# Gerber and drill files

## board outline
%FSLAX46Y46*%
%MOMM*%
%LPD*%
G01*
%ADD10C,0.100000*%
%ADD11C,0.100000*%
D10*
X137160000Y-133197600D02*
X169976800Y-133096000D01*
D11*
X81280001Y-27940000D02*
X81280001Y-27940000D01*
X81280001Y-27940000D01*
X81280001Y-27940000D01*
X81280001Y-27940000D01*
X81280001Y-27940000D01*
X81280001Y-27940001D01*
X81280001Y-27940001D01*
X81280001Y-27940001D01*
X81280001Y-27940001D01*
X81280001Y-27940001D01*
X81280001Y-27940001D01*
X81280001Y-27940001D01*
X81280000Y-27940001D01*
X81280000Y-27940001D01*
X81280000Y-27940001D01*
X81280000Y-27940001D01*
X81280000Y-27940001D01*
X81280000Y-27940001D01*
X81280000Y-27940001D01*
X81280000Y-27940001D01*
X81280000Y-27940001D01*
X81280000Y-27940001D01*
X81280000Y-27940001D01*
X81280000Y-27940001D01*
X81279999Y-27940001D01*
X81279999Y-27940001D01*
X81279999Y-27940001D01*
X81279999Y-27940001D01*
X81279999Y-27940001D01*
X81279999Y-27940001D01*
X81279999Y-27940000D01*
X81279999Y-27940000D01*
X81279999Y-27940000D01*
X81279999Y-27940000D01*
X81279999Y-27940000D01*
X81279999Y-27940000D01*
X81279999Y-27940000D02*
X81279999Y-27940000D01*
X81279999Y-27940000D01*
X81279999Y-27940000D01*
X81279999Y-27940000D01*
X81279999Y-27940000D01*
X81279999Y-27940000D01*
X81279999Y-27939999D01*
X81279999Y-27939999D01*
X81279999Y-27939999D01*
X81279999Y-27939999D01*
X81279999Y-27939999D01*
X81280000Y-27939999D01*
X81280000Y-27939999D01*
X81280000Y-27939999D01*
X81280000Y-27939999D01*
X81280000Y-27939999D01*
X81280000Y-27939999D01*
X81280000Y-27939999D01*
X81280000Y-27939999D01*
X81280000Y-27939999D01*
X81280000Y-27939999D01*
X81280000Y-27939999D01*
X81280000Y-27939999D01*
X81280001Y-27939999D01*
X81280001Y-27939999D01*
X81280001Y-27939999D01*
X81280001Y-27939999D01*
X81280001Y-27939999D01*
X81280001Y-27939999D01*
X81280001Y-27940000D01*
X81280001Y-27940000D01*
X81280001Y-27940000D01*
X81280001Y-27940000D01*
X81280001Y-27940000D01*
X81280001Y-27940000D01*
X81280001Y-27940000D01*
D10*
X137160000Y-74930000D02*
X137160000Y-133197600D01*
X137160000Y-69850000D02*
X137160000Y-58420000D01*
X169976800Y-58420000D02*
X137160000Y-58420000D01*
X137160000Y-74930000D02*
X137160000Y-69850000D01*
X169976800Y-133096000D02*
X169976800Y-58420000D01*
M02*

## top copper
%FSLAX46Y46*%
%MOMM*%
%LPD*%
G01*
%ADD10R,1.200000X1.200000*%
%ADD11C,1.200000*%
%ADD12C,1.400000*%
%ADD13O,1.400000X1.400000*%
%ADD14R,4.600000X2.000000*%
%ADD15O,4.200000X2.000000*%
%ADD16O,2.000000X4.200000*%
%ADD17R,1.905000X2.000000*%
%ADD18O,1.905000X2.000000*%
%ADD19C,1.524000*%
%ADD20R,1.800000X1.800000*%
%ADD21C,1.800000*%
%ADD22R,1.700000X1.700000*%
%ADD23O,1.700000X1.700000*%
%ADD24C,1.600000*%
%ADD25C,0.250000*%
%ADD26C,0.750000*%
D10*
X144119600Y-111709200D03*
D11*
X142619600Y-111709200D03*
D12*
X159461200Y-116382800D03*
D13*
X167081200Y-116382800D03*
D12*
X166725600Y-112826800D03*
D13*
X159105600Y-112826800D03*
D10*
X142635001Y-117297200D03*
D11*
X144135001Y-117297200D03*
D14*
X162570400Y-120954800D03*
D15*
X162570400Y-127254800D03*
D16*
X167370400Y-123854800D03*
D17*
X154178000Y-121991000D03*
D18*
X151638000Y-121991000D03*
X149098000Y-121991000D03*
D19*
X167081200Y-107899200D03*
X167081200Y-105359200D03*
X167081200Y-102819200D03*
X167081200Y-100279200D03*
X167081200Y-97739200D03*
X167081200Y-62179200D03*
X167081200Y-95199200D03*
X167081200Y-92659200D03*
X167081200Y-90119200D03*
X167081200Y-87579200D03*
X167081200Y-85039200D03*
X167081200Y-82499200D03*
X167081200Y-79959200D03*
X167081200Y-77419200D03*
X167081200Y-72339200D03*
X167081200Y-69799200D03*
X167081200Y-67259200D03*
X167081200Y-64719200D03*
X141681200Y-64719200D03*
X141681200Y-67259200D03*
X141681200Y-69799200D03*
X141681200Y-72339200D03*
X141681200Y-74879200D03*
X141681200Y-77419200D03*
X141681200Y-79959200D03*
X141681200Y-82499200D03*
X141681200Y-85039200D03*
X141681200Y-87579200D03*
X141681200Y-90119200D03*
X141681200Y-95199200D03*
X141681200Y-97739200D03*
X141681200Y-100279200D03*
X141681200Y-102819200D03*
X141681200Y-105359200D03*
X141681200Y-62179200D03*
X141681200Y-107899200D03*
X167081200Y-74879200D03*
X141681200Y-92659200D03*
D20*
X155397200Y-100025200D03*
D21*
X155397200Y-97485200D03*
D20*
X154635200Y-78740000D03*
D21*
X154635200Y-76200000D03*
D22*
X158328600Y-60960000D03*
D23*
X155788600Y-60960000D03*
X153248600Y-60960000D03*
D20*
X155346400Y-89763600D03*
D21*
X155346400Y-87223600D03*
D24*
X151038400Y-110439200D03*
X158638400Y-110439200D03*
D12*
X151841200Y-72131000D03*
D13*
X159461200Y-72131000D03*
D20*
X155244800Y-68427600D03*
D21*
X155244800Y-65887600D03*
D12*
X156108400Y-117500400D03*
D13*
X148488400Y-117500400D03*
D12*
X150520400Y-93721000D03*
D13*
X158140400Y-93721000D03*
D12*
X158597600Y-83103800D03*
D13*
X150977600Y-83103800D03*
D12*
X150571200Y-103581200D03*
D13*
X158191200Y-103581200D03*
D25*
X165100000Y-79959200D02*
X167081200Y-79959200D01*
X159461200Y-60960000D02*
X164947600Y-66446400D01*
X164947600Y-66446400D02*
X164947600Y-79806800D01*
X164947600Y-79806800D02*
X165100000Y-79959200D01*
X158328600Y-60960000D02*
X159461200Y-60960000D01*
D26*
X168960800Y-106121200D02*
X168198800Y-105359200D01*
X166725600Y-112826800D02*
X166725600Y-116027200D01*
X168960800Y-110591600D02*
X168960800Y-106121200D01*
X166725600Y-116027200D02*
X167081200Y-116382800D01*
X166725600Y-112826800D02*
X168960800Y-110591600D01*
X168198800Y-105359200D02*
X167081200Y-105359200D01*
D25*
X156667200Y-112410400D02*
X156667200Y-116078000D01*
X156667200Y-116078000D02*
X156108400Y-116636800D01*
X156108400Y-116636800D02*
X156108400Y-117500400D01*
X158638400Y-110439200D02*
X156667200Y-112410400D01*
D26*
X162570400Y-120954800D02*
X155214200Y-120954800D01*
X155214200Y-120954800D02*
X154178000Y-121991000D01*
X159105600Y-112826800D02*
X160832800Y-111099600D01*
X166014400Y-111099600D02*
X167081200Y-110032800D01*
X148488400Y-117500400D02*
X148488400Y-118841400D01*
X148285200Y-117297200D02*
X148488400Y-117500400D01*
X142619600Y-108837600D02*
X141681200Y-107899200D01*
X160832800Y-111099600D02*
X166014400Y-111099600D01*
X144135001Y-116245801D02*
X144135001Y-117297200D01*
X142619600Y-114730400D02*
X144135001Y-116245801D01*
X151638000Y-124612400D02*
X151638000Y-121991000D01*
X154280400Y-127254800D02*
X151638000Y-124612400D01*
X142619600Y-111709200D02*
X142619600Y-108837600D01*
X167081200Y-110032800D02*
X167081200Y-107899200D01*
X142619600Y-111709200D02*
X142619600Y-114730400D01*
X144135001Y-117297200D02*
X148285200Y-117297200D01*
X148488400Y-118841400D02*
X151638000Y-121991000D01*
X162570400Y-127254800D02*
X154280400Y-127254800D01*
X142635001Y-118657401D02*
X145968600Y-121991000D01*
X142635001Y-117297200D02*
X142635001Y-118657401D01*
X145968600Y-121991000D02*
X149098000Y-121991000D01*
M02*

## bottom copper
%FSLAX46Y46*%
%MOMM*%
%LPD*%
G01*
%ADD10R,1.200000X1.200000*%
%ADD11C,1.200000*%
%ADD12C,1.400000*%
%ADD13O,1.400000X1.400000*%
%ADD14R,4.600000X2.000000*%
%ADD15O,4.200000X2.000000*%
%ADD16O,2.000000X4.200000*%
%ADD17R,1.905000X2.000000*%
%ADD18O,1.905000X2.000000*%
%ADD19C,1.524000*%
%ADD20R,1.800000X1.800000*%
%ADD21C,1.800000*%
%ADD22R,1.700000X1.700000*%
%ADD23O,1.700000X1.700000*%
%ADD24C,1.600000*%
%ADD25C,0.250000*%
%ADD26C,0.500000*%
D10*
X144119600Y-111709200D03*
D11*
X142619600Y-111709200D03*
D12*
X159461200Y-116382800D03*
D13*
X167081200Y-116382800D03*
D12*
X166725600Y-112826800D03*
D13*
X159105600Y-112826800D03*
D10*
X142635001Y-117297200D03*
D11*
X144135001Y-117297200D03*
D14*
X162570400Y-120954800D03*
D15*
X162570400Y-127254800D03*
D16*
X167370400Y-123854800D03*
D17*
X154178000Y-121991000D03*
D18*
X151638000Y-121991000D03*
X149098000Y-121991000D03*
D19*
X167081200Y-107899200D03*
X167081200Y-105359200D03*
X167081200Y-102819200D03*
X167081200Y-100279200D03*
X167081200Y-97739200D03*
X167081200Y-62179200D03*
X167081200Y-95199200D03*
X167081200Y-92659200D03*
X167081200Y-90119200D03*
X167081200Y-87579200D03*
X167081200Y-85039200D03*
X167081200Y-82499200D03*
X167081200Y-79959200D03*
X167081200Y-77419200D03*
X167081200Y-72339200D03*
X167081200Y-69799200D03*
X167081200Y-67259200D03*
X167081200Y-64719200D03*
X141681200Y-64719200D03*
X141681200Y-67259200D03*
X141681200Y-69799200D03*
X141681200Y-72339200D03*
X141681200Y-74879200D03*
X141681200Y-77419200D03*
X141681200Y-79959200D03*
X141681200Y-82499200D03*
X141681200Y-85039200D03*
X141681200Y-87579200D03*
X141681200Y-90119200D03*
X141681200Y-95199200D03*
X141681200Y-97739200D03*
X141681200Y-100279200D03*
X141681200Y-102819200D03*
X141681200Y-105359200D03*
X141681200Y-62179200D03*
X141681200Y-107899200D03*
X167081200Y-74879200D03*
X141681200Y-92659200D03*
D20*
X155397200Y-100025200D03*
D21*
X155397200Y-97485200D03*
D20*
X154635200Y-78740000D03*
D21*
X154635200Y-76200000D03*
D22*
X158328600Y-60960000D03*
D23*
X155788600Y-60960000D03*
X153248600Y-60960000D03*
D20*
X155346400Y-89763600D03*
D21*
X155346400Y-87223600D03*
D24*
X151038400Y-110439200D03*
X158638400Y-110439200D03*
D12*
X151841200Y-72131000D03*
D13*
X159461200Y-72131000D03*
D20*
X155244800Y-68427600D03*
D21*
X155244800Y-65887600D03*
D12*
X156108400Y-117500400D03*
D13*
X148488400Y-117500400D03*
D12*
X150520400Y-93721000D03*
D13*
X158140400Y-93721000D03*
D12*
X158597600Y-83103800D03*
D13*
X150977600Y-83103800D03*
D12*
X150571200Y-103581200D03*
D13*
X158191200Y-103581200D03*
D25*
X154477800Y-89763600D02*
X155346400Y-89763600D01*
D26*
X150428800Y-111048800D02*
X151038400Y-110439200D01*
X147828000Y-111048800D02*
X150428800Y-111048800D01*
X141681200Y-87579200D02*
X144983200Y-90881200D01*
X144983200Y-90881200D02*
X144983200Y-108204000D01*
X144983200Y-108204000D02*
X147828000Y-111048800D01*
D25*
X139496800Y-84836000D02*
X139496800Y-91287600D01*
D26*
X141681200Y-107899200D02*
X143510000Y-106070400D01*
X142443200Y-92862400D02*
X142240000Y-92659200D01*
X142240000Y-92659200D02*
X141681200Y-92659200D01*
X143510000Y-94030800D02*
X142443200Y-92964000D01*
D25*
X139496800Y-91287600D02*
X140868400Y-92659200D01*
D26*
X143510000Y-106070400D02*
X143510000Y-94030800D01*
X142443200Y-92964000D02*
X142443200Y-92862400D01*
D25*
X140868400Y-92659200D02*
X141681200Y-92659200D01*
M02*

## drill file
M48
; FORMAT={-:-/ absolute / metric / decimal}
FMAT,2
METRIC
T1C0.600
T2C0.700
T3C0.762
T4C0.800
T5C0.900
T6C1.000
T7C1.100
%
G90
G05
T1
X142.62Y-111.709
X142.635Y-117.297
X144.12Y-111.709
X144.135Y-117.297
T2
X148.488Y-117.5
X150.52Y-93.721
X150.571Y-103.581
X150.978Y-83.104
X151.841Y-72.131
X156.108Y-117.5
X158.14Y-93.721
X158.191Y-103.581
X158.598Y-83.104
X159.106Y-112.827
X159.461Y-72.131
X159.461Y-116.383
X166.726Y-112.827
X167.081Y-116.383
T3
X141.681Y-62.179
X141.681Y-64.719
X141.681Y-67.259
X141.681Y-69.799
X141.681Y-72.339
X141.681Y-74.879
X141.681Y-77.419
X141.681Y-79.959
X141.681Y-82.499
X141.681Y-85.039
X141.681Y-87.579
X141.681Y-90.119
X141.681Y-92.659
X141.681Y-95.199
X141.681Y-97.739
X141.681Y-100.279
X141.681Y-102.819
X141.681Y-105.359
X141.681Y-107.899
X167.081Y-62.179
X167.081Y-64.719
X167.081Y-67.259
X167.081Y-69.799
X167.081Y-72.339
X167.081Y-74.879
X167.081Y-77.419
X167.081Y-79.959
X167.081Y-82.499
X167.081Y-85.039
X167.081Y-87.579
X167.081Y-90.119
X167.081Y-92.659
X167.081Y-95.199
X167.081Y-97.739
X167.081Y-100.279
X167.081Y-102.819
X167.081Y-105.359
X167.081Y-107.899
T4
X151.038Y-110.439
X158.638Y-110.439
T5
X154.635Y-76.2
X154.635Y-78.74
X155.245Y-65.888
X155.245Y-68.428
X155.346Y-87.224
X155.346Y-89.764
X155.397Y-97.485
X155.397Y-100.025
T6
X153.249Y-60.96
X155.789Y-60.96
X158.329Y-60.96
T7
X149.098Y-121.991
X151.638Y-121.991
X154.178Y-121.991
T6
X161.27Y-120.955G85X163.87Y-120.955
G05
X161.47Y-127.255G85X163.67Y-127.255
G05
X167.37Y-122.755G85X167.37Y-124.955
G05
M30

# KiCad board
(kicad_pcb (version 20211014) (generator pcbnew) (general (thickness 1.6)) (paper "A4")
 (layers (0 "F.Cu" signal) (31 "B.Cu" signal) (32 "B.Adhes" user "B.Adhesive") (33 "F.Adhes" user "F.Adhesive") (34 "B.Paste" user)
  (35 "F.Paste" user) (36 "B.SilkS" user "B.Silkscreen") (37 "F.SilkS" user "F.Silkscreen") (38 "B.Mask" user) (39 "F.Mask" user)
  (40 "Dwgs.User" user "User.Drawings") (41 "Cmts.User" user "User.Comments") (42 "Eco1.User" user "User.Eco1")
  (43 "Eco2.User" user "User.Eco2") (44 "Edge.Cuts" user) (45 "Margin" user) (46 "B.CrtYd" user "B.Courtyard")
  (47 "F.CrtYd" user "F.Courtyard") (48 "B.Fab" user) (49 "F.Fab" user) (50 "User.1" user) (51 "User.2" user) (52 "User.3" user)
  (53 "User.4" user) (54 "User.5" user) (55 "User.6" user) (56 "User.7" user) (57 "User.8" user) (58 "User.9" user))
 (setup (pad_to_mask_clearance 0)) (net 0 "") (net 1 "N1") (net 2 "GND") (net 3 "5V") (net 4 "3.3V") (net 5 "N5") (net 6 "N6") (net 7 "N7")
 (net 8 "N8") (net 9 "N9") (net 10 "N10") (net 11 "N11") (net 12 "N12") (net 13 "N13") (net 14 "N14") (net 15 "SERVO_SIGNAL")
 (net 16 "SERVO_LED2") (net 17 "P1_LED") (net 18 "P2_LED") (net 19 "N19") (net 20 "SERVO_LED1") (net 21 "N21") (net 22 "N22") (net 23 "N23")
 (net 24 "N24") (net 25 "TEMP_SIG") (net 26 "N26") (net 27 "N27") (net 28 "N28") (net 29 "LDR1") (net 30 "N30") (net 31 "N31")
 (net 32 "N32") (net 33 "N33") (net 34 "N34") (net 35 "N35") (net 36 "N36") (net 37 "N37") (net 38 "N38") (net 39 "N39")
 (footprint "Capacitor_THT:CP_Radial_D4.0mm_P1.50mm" (layer "F.Cu") (at 144.1196 111.7092 180)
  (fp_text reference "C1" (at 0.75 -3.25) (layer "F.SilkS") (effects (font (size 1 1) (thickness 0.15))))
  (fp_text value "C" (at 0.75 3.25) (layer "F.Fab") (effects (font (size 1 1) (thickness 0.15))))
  (pad "1" thru_hole rect (at 0 0 180) (size 1.2 1.2) (drill 0.6) (layers *.Cu *.Mask) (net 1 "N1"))
  (pad "2" thru_hole circle (at 1.5 0 180) (size 1.2 1.2) (drill 0.6) (layers *.Cu *.Mask) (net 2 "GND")))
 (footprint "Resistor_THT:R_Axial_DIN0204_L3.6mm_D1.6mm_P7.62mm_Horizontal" (layer "F.Cu") (at 159.4612 116.3828)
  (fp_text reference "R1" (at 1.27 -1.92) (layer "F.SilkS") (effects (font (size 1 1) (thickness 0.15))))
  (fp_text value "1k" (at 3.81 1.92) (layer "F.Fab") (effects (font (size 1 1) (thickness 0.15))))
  (pad "1" thru_hole circle (at 0 0) (size 1.4 1.4) (drill 0.7) (layers *.Cu *.Mask) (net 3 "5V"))
  (pad "2" thru_hole oval (at 7.62 0) (size 1.4 1.4) (drill 0.7) (layers *.Cu *.Mask) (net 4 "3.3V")))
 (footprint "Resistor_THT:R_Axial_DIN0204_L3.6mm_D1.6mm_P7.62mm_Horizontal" (layer "F.Cu") (at 166.7256 112.8268 180)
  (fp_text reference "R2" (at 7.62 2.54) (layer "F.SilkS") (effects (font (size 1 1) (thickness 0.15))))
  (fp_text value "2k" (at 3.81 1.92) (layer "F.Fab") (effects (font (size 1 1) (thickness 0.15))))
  (pad "1" thru_hole circle (at 0 0 180) (size 1.4 1.4) (drill 0.7) (layers *.Cu *.Mask) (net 4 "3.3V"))
  (pad "2" thru_hole oval (at 7.62 0 180) (size 1.4 1.4) (drill 0.7) (layers *.Cu *.Mask) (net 2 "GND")))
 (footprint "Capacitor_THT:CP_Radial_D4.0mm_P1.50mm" (layer "F.Cu") (at 142.635001 117.2972)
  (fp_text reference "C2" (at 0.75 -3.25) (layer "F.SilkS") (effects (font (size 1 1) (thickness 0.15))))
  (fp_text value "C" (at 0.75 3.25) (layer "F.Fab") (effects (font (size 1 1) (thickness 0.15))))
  (pad "1" thru_hole rect (at 0 0) (size 1.2 1.2) (drill 0.6) (layers *.Cu *.Mask) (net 3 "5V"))
  (pad "2" thru_hole circle (at 1.5 0) (size 1.2 1.2) (drill 0.6) (layers *.Cu *.Mask) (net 2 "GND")))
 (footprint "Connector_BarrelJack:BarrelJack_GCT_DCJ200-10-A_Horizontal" (layer "F.Cu") (at 162.5704 120.9548)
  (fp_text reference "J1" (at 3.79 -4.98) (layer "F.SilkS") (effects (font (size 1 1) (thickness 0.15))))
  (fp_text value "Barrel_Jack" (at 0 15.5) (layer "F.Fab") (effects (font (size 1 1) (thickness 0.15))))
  (pad "1" thru_hole rect (at 0 0) (size 4.6 2) (drill oval 3.6 1) (layers *.Cu *.Mask) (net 1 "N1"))
  (pad "2" thru_hole oval (at 0 6.3) (size 4.2 2) (drill oval 3.2 1) (layers *.Cu *.Mask) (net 2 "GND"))
  (pad "3" thru_hole oval (at 4.8 2.9) (size 2 4.2) (drill oval 1 3.2) (layers *.Cu *.Mask)))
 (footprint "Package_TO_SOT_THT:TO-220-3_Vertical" (layer "F.Cu") (at 154.178 121.991 180)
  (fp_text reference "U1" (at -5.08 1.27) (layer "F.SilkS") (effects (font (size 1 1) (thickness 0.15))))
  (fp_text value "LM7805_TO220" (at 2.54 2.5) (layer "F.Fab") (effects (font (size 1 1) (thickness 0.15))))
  (pad "1" thru_hole rect (at 0 0 180) (size 1.905 2) (drill 1.1) (layers *.Cu *.Mask) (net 1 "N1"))
  (pad "2" thru_hole oval (at 2.54 0 180) (size 1.905 2) (drill 1.1) (layers *.Cu *.Mask) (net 2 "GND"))
  (pad "3" thru_hole oval (at 5.08 0 180) (size 1.905 2) (drill 1.1) (layers *.Cu *.Mask) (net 3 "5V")))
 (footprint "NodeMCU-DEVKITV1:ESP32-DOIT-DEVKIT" (layer "F.Cu") (at 154.3812 110.4392 180)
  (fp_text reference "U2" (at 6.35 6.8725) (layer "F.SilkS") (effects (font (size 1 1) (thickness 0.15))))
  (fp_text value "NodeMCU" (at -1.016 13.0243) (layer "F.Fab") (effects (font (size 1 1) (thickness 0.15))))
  (pad "1" thru_hole circle (at -12.7 2.54 180) (size 1.524 1.524) (drill 0.762) (layers *.Cu *.Mask) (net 2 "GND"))
  (pad "2" thru_hole circle (at -12.7 5.08 180) (size 1.524 1.524) (drill 0.762) (layers *.Cu *.Mask) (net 4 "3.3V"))
  (pad "3" thru_hole circle (at -12.7 7.62 180) (size 1.524 1.524) (drill 0.762) (layers *.Cu *.Mask) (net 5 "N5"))
  (pad "4" thru_hole circle (at -12.7 10.16 180) (size 1.524 1.524) (drill 0.762) (layers *.Cu *.Mask) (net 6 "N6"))
  (pad "5" thru_hole circle (at -12.7 12.7 180) (size 1.524 1.524) (drill 0.762) (layers *.Cu *.Mask) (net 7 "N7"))
  (pad "5V" thru_hole circle (at -12.7 48.26 180) (size 1.524 1.524) (drill 0.762) (layers *.Cu *.Mask) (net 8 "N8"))
  (pad "6" thru_hole circle (at -12.7 15.24 180) (size 1.524 1.524) (drill 0.762) (layers *.Cu *.Mask) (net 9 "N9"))
  (pad "7" thru_hole circle (at -12.7 17.78 180) (size 1.524 1.524) (drill 0.762) (layers *.Cu *.Mask) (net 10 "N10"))
  (pad "8" thru_hole circle (at -12.7 20.32 180) (size 1.524 1.524) (drill 0.762) (layers *.Cu *.Mask) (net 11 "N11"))
  (pad "9" thru_hole circle (at -12.7 22.86 180) (size 1.524 1.524) (drill 0.762) (layers *.Cu *.Mask) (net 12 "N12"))
  (pad "10" thru_hole circle (at -12.7 25.4 180) (size 1.524 1.524) (drill 0.762) (layers *.Cu *.Mask) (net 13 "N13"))
  (pad "11" thru_hole circle (at -12.7 27.94 180) (size 1.524 1.524) (drill 0.762) (layers *.Cu *.Mask) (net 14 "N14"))
  (pad "12" thru_hole circle (at -12.7 30.48 180) (size 1.524 1.524) (drill 0.762) (layers *.Cu *.Mask) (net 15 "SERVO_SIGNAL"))
  (pad "13" thru_hole circle (at -12.7 33.02 180) (size 1.524 1.524) (drill 0.762) (layers *.Cu *.Mask) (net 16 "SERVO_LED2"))
  (pad "15" thru_hole circle (at -12.7 38.1 180) (size 1.524 1.524) (drill 0.762) (layers *.Cu *.Mask))
  (pad "16" thru_hole circle (at -12.7 40.64 180) (size 1.524 1.524) (drill 0.762) (layers *.Cu *.Mask) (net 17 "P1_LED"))
  (pad "17" thru_hole circle (at -12.7 43.18 180) (size 1.524 1.524) (drill 0.762) (layers *.Cu *.Mask) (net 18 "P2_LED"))
  (pad "18" thru_hole circle (at -12.7 45.72 180) (size 1.524 1.524) (drill 0.762) (layers *.Cu *.Mask) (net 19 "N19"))
  (pad "19" thru_hole circle (at 12.7 45.72 180) (size 1.524 1.524) (drill 0.762) (layers *.Cu *.Mask) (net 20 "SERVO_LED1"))
  (pad "20" thru_hole circle (at 12.7 43.18 180) (size 1.524 1.524) (drill 0.762) (layers *.Cu *.Mask) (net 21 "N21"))
  (pad "21" thru_hole circle (at 12.7 40.64 180) (size 1.524 1.524) (drill 0.762) (layers *.Cu *.Mask) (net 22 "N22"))
  (pad "22" thru_hole circle (at 12.7 38.1 180) (size 1.524 1.524) (drill 0.762) (layers *.Cu *.Mask) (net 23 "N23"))
  (pad "23" thru_hole circle (at 12.7 35.56 180) (size 1.524 1.524) (drill 0.762) (layers *.Cu *.Mask) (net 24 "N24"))
  (pad "24" thru_hole circle (at 12.7 33.02 180) (size 1.524 1.524) (drill 0.762) (layers *.Cu *.Mask) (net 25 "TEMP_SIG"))
  (pad "25" thru_hole circle (at 12.7 30.48 180) (size 1.524 1.524) (drill 0.762) (layers *.Cu *.Mask) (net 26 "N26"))
  (pad "26" thru_hole circle (at 12.7 27.94 180) (size 1.524 1.524) (drill 0.762) (layers *.Cu *.Mask) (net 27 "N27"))
  (pad "27" thru_hole circle (at 12.7 25.4 180) (size 1.524 1.524) (drill 0.762) (layers *.Cu *.Mask) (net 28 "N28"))
  (pad "28" thru_hole circle (at 12.7 22.86 180) (size 1.524 1.524) (drill 0.762) (layers *.Cu *.Mask) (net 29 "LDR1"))
  (pad "29" thru_hole circle (at 12.7 20.32 180) (size 1.524 1.524) (drill 0.762) (layers *.Cu *.Mask) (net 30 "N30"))
  (pad "31" thru_hole circle (at 12.7 15.24 180) (size 1.524 1.524) (drill 0.762) (layers *.Cu *.Mask) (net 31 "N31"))
  (pad "32" thru_hole circle (at 12.7 12.7 180) (size 1.524 1.524) (drill 0.762) (layers *.Cu *.Mask))
  (pad "33" thru_hole circle (at 12.7 10.16 180) (size 1.524 1.524) (drill 0.762) (layers *.Cu *.Mask) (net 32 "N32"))
  (pad "34" thru_hole circle (at 12.7 7.62 180) (size 1.524 1.524) (drill 0.762) (layers *.Cu *.Mask) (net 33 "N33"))
  (pad "35" thru_hole circle (at 12.7 5.08 180) (size 1.524 1.524) (drill 0.762) (layers *.Cu *.Mask) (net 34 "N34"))
  (pad "38" thru_hole circle (at 12.7 48.26 180) (size 1.524 1.524) (drill 0.762) (layers *.Cu *.Mask))
  (pad "GND" thru_hole circle (at 12.7 2.54 180) (size 1.524 1.524) (drill 0.762) (layers *.Cu *.Mask) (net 2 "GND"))
  (pad "GND" thru_hole circle (at -12.7 35.56 180) (size 1.524 1.524) (drill 0.762) (layers *.Cu *.Mask) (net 2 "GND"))
  (pad "GND" thru_hole circle (at 12.7 17.78 180) (size 1.524 1.524) (drill 0.762) (layers *.Cu *.Mask) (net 2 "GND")))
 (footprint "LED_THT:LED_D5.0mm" (layer "B.Cu") (at 155.3972 100.0252 90)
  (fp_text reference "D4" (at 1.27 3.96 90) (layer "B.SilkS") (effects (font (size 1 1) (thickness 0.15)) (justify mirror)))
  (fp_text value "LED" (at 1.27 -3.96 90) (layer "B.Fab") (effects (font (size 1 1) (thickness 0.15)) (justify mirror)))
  (pad "1" thru_hole rect (at 0 0 90) (size 1.8 1.8) (drill 0.9) (layers *.Cu *.Mask) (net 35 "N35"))
  (pad "2" thru_hole circle (at 2.54 0 90) (size 1.8 1.8) (drill 0.9) (layers *.Cu *.Mask) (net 18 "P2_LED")))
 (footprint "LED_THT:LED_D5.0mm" (layer "B.Cu") (at 154.6352 78.74 90)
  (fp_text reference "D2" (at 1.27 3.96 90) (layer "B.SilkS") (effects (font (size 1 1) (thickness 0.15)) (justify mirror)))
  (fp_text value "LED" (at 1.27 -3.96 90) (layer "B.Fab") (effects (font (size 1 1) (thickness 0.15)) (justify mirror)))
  (pad "1" thru_hole rect (at 0 0 90) (size 1.8 1.8) (drill 0.9) (layers *.Cu *.Mask) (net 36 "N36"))
  (pad "2" thru_hole circle (at 2.54 0 90) (size 1.8 1.8) (drill 0.9) (layers *.Cu *.Mask) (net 20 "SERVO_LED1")))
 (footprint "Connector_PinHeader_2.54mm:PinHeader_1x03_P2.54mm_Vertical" (layer "B.Cu") (at 158.3286 60.96 90)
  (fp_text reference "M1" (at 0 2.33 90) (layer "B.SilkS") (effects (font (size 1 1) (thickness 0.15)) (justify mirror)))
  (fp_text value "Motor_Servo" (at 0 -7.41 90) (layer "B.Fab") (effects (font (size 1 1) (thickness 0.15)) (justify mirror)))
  (pad "1" thru_hole rect (at 0 0 90) (size 1.7 1.7) (drill 1) (layers *.Cu *.Mask) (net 15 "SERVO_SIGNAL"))
  (pad "2" thru_hole oval (at 0 -2.54 90) (size 1.7 1.7) (drill 1) (layers *.Cu *.Mask) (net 3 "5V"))
  (pad "3" thru_hole oval (at 0 -5.08 90) (size 1.7 1.7) (drill 1) (layers *.Cu *.Mask) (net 2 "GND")))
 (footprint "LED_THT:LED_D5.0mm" (layer "B.Cu") (at 155.3464 89.7636 90)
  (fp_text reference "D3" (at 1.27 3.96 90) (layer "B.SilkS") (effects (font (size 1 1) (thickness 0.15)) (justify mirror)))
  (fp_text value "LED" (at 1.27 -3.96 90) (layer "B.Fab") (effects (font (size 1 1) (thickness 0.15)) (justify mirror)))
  (pad "1" thru_hole rect (at 0 0 90) (size 1.8 1.8) (drill 0.9) (layers *.Cu *.Mask) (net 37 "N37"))
  (pad "2" thru_hole circle (at 2.54 0 90) (size 1.8 1.8) (drill 0.9) (layers *.Cu *.Mask) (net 17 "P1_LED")))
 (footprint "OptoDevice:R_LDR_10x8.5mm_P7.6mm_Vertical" (layer "B.Cu") (at 151.0384 110.4392)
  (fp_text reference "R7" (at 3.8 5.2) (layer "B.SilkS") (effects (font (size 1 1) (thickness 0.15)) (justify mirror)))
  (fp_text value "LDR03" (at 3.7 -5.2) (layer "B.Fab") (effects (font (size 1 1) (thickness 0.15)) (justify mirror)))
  (pad "1" thru_hole circle (at 0 0) (size 1.6 1.6) (drill 0.8) (layers *.Cu *.Mask) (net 29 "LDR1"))
  (pad "2" thru_hole circle (at 7.6 0) (size 1.6 1.6) (drill 0.8) (layers *.Cu *.Mask) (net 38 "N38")))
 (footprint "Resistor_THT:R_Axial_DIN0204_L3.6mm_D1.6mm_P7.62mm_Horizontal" (layer "B.Cu") (at 151.8412 72.131)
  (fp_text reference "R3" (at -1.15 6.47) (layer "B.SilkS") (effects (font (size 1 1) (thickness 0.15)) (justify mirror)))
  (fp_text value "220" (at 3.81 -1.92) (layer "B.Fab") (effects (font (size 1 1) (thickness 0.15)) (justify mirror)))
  (pad "1" thru_hole circle (at 0 0) (size 1.4 1.4) (drill 0.7) (layers *.Cu *.Mask) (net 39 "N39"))
  (pad "2" thru_hole oval (at 7.62 0) (size 1.4 1.4) (drill 0.7) (layers *.Cu *.Mask) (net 2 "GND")))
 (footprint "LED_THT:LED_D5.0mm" (layer "B.Cu") (at 155.2448 68.4276 90)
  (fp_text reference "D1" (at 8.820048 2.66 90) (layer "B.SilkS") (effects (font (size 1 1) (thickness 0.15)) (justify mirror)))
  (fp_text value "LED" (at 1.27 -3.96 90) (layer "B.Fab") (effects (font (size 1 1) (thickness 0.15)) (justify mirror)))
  (pad "1" thru_hole rect (at 0 0 90) (size 1.8 1.8) (drill 0.9) (layers *.Cu *.Mask) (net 39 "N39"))
  (pad "2" thru_hole circle (at 2.54 0 90) (size 1.8 1.8) (drill 0.9) (layers *.Cu *.Mask) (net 16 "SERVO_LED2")))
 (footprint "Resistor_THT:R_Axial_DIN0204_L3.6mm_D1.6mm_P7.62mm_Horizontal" (layer "B.Cu") (at 156.1084 117.5004 180)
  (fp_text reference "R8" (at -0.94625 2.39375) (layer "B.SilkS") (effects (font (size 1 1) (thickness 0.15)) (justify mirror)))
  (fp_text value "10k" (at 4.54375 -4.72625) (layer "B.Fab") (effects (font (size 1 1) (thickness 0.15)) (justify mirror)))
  (pad "1" thru_hole circle (at 0 0 180) (size 1.4 1.4) (drill 0.7) (layers *.Cu *.Mask) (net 38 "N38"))
  (pad "2" thru_hole oval (at 7.62 0 180) (size 1.4 1.4) (drill 0.7) (layers *.Cu *.Mask) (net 2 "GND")))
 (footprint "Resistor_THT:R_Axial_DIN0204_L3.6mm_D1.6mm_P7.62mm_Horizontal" (layer "B.Cu") (at 150.5204 93.721)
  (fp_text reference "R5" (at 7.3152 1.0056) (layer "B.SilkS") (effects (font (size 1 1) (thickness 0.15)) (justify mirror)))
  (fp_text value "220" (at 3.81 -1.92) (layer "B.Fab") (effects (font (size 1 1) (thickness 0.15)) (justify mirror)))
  (pad "1" thru_hole circle (at 0 0) (size 1.4 1.4) (drill 0.7) (layers *.Cu *.Mask) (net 37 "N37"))
  (pad "2" thru_hole oval (at 7.62 0) (size 1.4 1.4) (drill 0.7) (layers *.Cu *.Mask) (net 2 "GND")))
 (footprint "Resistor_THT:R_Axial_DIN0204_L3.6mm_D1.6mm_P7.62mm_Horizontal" (layer "B.Cu") (at 158.5976 83.1038 180)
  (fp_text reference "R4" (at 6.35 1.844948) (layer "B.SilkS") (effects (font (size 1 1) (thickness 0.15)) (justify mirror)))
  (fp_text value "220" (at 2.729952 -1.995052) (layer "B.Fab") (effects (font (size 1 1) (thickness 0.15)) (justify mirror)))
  (pad "1" thru_hole circle (at 0 0 180) (size 1.4 1.4) (drill 0.7) (layers *.Cu *.Mask) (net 36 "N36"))
  (pad "2" thru_hole oval (at 7.62 0 180) (size 1.4 1.4) (drill 0.7) (layers *.Cu *.Mask) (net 2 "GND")))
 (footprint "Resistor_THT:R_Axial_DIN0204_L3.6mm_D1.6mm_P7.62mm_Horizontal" (layer "B.Cu") (at 150.5712 103.5812)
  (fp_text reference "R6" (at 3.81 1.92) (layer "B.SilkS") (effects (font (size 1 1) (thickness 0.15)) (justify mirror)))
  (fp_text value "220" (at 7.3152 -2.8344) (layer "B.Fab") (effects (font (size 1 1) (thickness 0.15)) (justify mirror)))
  (pad "1" thru_hole circle (at 0 0) (size 1.4 1.4) (drill 0.7) (layers *.Cu *.Mask) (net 35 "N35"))
  (pad "2" thru_hole oval (at 7.62 0) (size 1.4 1.4) (drill 0.7) (layers *.Cu *.Mask) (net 2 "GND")))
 (gr_line (start 137.16 133.1976) (end 169.9768 133.096) (layer "Edge.Cuts") (width 0.1))
 (gr_arc (start 81.28 27.94) (mid 81.28 27.94) (end 81.28 27.94) (layer "Edge.Cuts") (width 0.1))
 (gr_line (start 137.16 74.93) (end 137.16 133.1976) (layer "Edge.Cuts") (width 0.1))
 (gr_line (start 137.16 69.85) (end 137.16 58.42) (layer "Edge.Cuts") (width 0.1))
 (gr_line (start 169.9768 58.42) (end 137.16 58.42) (layer "Edge.Cuts") (width 0.1))
 (gr_line (start 137.16 74.93) (end 137.16 69.85) (layer "Edge.Cuts") (width 0.1))
 (gr_line (start 169.9768 133.096) (end 169.9768 58.42) (layer "Edge.Cuts") (width 0.1))
 (segment (start 154.4778 89.7636) (end 155.3464 89.7636) (width 0.25) (layer "B.Cu") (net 37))
 (segment (start 165.1 79.9592) (end 167.0812 79.9592) (width 0.25) (layer "F.Cu") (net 15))
 (segment (start 159.4612 60.96) (end 164.9476 66.4464) (width 0.25) (layer "F.Cu") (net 15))
 (segment (start 164.9476 66.4464) (end 164.9476 79.8068) (width 0.25) (layer "F.Cu") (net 15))
 (segment (start 164.9476 79.8068) (end 165.1 79.9592) (width 0.25) (layer "F.Cu") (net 15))
 (segment (start 158.3286 60.96) (end 159.4612 60.96) (width 0.25) (layer "F.Cu") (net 15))
 (segment (start 168.9608 106.1212) (end 168.1988 105.3592) (width 0.75) (layer "F.Cu") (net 4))
 (segment (start 166.7256 112.8268) (end 166.7256 116.0272) (width 0.75) (layer "F.Cu") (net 4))
 (segment (start 168.9608 110.5916) (end 168.9608 106.1212) (width 0.75) (layer "F.Cu") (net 4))
 (segment (start 166.7256 116.0272) (end 167.0812 116.3828) (width 0.75) (layer "F.Cu") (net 4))
 (segment (start 166.7256 112.8268) (end 168.9608 110.5916) (width 0.75) (layer "F.Cu") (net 4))
 (segment (start 168.1988 105.3592) (end 167.0812 105.3592) (width 0.75) (layer "F.Cu") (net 4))
 (segment (start 150.4288 111.0488) (end 151.0384 110.4392) (width 0.5) (layer "B.Cu") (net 29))
 (segment (start 147.828 111.0488) (end 150.4288 111.0488) (width 0.5) (layer "B.Cu") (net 29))
 (segment (start 141.6812 87.5792) (end 144.9832 90.8812) (width 0.5) (layer "B.Cu") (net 29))
 (segment (start 144.9832 90.8812) (end 144.9832 108.204) (width 0.5) (layer "B.Cu") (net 29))
 (segment (start 144.9832 108.204) (end 147.828 111.0488) (width 0.5) (layer "B.Cu") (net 29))
 (segment (start 156.6672 112.4104) (end 156.6672 116.078) (width 0.25) (layer "F.Cu") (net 38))
 (segment (start 156.6672 116.078) (end 156.1084 116.6368) (width 0.25) (layer "F.Cu") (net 38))
 (segment (start 156.1084 116.6368) (end 156.1084 117.5004) (width 0.25) (layer "F.Cu") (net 38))
 (segment (start 158.6384 110.4392) (end 156.6672 112.4104) (width 0.25) (layer "F.Cu") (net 38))
 (segment (start 162.5704 120.9548) (end 155.2142 120.9548) (width 0.75) (layer "F.Cu") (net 1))
 (segment (start 155.2142 120.9548) (end 154.178 121.991) (width 0.75) (layer "F.Cu") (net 1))
 (segment (start 159.1056 112.8268) (end 160.8328 111.0996) (width 0.75) (layer "F.Cu") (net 2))
 (segment (start 166.0144 111.0996) (end 167.0812 110.0328) (width 0.75) (layer "F.Cu") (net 2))
 (segment (start 148.4884 117.5004) (end 148.4884 118.8414) (width 0.75) (layer "F.Cu") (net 2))
 (segment (start 148.2852 117.2972) (end 148.4884 117.5004) (width 0.75) (layer "F.Cu") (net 2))
 (segment (start 142.6196 108.8376) (end 141.6812 107.8992) (width 0.75) (layer "F.Cu") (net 2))
 (segment (start 160.8328 111.0996) (end 166.0144 111.0996) (width 0.75) (layer "F.Cu") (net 2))
 (segment (start 144.135001 116.245801) (end 144.135001 117.2972) (width 0.75) (layer "F.Cu") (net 2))
 (segment (start 142.6196 114.7304) (end 144.135001 116.245801) (width 0.75) (layer "F.Cu") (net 2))
 (segment (start 151.638 124.6124) (end 151.638 121.991) (width 0.75) (layer "F.Cu") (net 2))
 (segment (start 154.2804 127.2548) (end 151.638 124.6124) (width 0.75) (layer "F.Cu") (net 2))
 (segment (start 142.6196 111.7092) (end 142.6196 108.8376) (width 0.75) (layer "F.Cu") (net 2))
 (segment (start 167.0812 110.0328) (end 167.0812 107.8992) (width 0.75) (layer "F.Cu") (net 2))
 (segment (start 142.6196 111.7092) (end 142.6196 114.7304) (width 0.75) (layer "F.Cu") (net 2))
 (segment (start 144.135001 117.2972) (end 148.2852 117.2972) (width 0.75) (layer "F.Cu") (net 2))
 (segment (start 148.4884 118.8414) (end 151.638 121.991) (width 0.75) (layer "F.Cu") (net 2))
 (segment (start 162.5704 127.2548) (end 154.2804 127.2548) (width 0.75) (layer "F.Cu") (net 2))
 (segment (start 139.4968 84.836) (end 139.4968 91.2876) (width 0.25) (layer "B.Cu") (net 2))
 (segment (start 141.6812 107.8992) (end 143.51 106.0704) (width 0.5) (layer "B.Cu") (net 2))
 (segment (start 142.4432 92.8624) (end 142.24 92.6592) (width 0.5) (layer "B.Cu") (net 2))
 (segment (start 142.24 92.6592) (end 141.6812 92.6592) (width 0.5) (layer "B.Cu") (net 2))
 (segment (start 143.51 94.0308) (end 142.4432 92.964) (width 0.5) (layer "B.Cu") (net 2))
 (segment (start 139.4968 91.2876) (end 140.8684 92.6592) (width 0.25) (layer "B.Cu") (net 2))
 (segment (start 143.51 106.0704) (end 143.51 94.0308) (width 0.5) (layer "B.Cu") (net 2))
 (segment (start 142.4432 92.964) (end 142.4432 92.8624) (width 0.5) (layer "B.Cu") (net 2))
 (segment (start 140.8684 92.6592) (end 141.6812 92.6592) (width 0.25) (layer "B.Cu") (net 2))
 (segment (start 142.635001 118.657401) (end 145.9686 121.991) (width 0.75) (layer "F.Cu") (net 3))
 (segment (start 142.635001 117.2972) (end 142.635001 118.657401) (width 0.75) (layer "F.Cu") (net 3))
 (segment (start 145.9686 121.991) (end 149.098 121.991) (width 0.75) (layer "F.Cu") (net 3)))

